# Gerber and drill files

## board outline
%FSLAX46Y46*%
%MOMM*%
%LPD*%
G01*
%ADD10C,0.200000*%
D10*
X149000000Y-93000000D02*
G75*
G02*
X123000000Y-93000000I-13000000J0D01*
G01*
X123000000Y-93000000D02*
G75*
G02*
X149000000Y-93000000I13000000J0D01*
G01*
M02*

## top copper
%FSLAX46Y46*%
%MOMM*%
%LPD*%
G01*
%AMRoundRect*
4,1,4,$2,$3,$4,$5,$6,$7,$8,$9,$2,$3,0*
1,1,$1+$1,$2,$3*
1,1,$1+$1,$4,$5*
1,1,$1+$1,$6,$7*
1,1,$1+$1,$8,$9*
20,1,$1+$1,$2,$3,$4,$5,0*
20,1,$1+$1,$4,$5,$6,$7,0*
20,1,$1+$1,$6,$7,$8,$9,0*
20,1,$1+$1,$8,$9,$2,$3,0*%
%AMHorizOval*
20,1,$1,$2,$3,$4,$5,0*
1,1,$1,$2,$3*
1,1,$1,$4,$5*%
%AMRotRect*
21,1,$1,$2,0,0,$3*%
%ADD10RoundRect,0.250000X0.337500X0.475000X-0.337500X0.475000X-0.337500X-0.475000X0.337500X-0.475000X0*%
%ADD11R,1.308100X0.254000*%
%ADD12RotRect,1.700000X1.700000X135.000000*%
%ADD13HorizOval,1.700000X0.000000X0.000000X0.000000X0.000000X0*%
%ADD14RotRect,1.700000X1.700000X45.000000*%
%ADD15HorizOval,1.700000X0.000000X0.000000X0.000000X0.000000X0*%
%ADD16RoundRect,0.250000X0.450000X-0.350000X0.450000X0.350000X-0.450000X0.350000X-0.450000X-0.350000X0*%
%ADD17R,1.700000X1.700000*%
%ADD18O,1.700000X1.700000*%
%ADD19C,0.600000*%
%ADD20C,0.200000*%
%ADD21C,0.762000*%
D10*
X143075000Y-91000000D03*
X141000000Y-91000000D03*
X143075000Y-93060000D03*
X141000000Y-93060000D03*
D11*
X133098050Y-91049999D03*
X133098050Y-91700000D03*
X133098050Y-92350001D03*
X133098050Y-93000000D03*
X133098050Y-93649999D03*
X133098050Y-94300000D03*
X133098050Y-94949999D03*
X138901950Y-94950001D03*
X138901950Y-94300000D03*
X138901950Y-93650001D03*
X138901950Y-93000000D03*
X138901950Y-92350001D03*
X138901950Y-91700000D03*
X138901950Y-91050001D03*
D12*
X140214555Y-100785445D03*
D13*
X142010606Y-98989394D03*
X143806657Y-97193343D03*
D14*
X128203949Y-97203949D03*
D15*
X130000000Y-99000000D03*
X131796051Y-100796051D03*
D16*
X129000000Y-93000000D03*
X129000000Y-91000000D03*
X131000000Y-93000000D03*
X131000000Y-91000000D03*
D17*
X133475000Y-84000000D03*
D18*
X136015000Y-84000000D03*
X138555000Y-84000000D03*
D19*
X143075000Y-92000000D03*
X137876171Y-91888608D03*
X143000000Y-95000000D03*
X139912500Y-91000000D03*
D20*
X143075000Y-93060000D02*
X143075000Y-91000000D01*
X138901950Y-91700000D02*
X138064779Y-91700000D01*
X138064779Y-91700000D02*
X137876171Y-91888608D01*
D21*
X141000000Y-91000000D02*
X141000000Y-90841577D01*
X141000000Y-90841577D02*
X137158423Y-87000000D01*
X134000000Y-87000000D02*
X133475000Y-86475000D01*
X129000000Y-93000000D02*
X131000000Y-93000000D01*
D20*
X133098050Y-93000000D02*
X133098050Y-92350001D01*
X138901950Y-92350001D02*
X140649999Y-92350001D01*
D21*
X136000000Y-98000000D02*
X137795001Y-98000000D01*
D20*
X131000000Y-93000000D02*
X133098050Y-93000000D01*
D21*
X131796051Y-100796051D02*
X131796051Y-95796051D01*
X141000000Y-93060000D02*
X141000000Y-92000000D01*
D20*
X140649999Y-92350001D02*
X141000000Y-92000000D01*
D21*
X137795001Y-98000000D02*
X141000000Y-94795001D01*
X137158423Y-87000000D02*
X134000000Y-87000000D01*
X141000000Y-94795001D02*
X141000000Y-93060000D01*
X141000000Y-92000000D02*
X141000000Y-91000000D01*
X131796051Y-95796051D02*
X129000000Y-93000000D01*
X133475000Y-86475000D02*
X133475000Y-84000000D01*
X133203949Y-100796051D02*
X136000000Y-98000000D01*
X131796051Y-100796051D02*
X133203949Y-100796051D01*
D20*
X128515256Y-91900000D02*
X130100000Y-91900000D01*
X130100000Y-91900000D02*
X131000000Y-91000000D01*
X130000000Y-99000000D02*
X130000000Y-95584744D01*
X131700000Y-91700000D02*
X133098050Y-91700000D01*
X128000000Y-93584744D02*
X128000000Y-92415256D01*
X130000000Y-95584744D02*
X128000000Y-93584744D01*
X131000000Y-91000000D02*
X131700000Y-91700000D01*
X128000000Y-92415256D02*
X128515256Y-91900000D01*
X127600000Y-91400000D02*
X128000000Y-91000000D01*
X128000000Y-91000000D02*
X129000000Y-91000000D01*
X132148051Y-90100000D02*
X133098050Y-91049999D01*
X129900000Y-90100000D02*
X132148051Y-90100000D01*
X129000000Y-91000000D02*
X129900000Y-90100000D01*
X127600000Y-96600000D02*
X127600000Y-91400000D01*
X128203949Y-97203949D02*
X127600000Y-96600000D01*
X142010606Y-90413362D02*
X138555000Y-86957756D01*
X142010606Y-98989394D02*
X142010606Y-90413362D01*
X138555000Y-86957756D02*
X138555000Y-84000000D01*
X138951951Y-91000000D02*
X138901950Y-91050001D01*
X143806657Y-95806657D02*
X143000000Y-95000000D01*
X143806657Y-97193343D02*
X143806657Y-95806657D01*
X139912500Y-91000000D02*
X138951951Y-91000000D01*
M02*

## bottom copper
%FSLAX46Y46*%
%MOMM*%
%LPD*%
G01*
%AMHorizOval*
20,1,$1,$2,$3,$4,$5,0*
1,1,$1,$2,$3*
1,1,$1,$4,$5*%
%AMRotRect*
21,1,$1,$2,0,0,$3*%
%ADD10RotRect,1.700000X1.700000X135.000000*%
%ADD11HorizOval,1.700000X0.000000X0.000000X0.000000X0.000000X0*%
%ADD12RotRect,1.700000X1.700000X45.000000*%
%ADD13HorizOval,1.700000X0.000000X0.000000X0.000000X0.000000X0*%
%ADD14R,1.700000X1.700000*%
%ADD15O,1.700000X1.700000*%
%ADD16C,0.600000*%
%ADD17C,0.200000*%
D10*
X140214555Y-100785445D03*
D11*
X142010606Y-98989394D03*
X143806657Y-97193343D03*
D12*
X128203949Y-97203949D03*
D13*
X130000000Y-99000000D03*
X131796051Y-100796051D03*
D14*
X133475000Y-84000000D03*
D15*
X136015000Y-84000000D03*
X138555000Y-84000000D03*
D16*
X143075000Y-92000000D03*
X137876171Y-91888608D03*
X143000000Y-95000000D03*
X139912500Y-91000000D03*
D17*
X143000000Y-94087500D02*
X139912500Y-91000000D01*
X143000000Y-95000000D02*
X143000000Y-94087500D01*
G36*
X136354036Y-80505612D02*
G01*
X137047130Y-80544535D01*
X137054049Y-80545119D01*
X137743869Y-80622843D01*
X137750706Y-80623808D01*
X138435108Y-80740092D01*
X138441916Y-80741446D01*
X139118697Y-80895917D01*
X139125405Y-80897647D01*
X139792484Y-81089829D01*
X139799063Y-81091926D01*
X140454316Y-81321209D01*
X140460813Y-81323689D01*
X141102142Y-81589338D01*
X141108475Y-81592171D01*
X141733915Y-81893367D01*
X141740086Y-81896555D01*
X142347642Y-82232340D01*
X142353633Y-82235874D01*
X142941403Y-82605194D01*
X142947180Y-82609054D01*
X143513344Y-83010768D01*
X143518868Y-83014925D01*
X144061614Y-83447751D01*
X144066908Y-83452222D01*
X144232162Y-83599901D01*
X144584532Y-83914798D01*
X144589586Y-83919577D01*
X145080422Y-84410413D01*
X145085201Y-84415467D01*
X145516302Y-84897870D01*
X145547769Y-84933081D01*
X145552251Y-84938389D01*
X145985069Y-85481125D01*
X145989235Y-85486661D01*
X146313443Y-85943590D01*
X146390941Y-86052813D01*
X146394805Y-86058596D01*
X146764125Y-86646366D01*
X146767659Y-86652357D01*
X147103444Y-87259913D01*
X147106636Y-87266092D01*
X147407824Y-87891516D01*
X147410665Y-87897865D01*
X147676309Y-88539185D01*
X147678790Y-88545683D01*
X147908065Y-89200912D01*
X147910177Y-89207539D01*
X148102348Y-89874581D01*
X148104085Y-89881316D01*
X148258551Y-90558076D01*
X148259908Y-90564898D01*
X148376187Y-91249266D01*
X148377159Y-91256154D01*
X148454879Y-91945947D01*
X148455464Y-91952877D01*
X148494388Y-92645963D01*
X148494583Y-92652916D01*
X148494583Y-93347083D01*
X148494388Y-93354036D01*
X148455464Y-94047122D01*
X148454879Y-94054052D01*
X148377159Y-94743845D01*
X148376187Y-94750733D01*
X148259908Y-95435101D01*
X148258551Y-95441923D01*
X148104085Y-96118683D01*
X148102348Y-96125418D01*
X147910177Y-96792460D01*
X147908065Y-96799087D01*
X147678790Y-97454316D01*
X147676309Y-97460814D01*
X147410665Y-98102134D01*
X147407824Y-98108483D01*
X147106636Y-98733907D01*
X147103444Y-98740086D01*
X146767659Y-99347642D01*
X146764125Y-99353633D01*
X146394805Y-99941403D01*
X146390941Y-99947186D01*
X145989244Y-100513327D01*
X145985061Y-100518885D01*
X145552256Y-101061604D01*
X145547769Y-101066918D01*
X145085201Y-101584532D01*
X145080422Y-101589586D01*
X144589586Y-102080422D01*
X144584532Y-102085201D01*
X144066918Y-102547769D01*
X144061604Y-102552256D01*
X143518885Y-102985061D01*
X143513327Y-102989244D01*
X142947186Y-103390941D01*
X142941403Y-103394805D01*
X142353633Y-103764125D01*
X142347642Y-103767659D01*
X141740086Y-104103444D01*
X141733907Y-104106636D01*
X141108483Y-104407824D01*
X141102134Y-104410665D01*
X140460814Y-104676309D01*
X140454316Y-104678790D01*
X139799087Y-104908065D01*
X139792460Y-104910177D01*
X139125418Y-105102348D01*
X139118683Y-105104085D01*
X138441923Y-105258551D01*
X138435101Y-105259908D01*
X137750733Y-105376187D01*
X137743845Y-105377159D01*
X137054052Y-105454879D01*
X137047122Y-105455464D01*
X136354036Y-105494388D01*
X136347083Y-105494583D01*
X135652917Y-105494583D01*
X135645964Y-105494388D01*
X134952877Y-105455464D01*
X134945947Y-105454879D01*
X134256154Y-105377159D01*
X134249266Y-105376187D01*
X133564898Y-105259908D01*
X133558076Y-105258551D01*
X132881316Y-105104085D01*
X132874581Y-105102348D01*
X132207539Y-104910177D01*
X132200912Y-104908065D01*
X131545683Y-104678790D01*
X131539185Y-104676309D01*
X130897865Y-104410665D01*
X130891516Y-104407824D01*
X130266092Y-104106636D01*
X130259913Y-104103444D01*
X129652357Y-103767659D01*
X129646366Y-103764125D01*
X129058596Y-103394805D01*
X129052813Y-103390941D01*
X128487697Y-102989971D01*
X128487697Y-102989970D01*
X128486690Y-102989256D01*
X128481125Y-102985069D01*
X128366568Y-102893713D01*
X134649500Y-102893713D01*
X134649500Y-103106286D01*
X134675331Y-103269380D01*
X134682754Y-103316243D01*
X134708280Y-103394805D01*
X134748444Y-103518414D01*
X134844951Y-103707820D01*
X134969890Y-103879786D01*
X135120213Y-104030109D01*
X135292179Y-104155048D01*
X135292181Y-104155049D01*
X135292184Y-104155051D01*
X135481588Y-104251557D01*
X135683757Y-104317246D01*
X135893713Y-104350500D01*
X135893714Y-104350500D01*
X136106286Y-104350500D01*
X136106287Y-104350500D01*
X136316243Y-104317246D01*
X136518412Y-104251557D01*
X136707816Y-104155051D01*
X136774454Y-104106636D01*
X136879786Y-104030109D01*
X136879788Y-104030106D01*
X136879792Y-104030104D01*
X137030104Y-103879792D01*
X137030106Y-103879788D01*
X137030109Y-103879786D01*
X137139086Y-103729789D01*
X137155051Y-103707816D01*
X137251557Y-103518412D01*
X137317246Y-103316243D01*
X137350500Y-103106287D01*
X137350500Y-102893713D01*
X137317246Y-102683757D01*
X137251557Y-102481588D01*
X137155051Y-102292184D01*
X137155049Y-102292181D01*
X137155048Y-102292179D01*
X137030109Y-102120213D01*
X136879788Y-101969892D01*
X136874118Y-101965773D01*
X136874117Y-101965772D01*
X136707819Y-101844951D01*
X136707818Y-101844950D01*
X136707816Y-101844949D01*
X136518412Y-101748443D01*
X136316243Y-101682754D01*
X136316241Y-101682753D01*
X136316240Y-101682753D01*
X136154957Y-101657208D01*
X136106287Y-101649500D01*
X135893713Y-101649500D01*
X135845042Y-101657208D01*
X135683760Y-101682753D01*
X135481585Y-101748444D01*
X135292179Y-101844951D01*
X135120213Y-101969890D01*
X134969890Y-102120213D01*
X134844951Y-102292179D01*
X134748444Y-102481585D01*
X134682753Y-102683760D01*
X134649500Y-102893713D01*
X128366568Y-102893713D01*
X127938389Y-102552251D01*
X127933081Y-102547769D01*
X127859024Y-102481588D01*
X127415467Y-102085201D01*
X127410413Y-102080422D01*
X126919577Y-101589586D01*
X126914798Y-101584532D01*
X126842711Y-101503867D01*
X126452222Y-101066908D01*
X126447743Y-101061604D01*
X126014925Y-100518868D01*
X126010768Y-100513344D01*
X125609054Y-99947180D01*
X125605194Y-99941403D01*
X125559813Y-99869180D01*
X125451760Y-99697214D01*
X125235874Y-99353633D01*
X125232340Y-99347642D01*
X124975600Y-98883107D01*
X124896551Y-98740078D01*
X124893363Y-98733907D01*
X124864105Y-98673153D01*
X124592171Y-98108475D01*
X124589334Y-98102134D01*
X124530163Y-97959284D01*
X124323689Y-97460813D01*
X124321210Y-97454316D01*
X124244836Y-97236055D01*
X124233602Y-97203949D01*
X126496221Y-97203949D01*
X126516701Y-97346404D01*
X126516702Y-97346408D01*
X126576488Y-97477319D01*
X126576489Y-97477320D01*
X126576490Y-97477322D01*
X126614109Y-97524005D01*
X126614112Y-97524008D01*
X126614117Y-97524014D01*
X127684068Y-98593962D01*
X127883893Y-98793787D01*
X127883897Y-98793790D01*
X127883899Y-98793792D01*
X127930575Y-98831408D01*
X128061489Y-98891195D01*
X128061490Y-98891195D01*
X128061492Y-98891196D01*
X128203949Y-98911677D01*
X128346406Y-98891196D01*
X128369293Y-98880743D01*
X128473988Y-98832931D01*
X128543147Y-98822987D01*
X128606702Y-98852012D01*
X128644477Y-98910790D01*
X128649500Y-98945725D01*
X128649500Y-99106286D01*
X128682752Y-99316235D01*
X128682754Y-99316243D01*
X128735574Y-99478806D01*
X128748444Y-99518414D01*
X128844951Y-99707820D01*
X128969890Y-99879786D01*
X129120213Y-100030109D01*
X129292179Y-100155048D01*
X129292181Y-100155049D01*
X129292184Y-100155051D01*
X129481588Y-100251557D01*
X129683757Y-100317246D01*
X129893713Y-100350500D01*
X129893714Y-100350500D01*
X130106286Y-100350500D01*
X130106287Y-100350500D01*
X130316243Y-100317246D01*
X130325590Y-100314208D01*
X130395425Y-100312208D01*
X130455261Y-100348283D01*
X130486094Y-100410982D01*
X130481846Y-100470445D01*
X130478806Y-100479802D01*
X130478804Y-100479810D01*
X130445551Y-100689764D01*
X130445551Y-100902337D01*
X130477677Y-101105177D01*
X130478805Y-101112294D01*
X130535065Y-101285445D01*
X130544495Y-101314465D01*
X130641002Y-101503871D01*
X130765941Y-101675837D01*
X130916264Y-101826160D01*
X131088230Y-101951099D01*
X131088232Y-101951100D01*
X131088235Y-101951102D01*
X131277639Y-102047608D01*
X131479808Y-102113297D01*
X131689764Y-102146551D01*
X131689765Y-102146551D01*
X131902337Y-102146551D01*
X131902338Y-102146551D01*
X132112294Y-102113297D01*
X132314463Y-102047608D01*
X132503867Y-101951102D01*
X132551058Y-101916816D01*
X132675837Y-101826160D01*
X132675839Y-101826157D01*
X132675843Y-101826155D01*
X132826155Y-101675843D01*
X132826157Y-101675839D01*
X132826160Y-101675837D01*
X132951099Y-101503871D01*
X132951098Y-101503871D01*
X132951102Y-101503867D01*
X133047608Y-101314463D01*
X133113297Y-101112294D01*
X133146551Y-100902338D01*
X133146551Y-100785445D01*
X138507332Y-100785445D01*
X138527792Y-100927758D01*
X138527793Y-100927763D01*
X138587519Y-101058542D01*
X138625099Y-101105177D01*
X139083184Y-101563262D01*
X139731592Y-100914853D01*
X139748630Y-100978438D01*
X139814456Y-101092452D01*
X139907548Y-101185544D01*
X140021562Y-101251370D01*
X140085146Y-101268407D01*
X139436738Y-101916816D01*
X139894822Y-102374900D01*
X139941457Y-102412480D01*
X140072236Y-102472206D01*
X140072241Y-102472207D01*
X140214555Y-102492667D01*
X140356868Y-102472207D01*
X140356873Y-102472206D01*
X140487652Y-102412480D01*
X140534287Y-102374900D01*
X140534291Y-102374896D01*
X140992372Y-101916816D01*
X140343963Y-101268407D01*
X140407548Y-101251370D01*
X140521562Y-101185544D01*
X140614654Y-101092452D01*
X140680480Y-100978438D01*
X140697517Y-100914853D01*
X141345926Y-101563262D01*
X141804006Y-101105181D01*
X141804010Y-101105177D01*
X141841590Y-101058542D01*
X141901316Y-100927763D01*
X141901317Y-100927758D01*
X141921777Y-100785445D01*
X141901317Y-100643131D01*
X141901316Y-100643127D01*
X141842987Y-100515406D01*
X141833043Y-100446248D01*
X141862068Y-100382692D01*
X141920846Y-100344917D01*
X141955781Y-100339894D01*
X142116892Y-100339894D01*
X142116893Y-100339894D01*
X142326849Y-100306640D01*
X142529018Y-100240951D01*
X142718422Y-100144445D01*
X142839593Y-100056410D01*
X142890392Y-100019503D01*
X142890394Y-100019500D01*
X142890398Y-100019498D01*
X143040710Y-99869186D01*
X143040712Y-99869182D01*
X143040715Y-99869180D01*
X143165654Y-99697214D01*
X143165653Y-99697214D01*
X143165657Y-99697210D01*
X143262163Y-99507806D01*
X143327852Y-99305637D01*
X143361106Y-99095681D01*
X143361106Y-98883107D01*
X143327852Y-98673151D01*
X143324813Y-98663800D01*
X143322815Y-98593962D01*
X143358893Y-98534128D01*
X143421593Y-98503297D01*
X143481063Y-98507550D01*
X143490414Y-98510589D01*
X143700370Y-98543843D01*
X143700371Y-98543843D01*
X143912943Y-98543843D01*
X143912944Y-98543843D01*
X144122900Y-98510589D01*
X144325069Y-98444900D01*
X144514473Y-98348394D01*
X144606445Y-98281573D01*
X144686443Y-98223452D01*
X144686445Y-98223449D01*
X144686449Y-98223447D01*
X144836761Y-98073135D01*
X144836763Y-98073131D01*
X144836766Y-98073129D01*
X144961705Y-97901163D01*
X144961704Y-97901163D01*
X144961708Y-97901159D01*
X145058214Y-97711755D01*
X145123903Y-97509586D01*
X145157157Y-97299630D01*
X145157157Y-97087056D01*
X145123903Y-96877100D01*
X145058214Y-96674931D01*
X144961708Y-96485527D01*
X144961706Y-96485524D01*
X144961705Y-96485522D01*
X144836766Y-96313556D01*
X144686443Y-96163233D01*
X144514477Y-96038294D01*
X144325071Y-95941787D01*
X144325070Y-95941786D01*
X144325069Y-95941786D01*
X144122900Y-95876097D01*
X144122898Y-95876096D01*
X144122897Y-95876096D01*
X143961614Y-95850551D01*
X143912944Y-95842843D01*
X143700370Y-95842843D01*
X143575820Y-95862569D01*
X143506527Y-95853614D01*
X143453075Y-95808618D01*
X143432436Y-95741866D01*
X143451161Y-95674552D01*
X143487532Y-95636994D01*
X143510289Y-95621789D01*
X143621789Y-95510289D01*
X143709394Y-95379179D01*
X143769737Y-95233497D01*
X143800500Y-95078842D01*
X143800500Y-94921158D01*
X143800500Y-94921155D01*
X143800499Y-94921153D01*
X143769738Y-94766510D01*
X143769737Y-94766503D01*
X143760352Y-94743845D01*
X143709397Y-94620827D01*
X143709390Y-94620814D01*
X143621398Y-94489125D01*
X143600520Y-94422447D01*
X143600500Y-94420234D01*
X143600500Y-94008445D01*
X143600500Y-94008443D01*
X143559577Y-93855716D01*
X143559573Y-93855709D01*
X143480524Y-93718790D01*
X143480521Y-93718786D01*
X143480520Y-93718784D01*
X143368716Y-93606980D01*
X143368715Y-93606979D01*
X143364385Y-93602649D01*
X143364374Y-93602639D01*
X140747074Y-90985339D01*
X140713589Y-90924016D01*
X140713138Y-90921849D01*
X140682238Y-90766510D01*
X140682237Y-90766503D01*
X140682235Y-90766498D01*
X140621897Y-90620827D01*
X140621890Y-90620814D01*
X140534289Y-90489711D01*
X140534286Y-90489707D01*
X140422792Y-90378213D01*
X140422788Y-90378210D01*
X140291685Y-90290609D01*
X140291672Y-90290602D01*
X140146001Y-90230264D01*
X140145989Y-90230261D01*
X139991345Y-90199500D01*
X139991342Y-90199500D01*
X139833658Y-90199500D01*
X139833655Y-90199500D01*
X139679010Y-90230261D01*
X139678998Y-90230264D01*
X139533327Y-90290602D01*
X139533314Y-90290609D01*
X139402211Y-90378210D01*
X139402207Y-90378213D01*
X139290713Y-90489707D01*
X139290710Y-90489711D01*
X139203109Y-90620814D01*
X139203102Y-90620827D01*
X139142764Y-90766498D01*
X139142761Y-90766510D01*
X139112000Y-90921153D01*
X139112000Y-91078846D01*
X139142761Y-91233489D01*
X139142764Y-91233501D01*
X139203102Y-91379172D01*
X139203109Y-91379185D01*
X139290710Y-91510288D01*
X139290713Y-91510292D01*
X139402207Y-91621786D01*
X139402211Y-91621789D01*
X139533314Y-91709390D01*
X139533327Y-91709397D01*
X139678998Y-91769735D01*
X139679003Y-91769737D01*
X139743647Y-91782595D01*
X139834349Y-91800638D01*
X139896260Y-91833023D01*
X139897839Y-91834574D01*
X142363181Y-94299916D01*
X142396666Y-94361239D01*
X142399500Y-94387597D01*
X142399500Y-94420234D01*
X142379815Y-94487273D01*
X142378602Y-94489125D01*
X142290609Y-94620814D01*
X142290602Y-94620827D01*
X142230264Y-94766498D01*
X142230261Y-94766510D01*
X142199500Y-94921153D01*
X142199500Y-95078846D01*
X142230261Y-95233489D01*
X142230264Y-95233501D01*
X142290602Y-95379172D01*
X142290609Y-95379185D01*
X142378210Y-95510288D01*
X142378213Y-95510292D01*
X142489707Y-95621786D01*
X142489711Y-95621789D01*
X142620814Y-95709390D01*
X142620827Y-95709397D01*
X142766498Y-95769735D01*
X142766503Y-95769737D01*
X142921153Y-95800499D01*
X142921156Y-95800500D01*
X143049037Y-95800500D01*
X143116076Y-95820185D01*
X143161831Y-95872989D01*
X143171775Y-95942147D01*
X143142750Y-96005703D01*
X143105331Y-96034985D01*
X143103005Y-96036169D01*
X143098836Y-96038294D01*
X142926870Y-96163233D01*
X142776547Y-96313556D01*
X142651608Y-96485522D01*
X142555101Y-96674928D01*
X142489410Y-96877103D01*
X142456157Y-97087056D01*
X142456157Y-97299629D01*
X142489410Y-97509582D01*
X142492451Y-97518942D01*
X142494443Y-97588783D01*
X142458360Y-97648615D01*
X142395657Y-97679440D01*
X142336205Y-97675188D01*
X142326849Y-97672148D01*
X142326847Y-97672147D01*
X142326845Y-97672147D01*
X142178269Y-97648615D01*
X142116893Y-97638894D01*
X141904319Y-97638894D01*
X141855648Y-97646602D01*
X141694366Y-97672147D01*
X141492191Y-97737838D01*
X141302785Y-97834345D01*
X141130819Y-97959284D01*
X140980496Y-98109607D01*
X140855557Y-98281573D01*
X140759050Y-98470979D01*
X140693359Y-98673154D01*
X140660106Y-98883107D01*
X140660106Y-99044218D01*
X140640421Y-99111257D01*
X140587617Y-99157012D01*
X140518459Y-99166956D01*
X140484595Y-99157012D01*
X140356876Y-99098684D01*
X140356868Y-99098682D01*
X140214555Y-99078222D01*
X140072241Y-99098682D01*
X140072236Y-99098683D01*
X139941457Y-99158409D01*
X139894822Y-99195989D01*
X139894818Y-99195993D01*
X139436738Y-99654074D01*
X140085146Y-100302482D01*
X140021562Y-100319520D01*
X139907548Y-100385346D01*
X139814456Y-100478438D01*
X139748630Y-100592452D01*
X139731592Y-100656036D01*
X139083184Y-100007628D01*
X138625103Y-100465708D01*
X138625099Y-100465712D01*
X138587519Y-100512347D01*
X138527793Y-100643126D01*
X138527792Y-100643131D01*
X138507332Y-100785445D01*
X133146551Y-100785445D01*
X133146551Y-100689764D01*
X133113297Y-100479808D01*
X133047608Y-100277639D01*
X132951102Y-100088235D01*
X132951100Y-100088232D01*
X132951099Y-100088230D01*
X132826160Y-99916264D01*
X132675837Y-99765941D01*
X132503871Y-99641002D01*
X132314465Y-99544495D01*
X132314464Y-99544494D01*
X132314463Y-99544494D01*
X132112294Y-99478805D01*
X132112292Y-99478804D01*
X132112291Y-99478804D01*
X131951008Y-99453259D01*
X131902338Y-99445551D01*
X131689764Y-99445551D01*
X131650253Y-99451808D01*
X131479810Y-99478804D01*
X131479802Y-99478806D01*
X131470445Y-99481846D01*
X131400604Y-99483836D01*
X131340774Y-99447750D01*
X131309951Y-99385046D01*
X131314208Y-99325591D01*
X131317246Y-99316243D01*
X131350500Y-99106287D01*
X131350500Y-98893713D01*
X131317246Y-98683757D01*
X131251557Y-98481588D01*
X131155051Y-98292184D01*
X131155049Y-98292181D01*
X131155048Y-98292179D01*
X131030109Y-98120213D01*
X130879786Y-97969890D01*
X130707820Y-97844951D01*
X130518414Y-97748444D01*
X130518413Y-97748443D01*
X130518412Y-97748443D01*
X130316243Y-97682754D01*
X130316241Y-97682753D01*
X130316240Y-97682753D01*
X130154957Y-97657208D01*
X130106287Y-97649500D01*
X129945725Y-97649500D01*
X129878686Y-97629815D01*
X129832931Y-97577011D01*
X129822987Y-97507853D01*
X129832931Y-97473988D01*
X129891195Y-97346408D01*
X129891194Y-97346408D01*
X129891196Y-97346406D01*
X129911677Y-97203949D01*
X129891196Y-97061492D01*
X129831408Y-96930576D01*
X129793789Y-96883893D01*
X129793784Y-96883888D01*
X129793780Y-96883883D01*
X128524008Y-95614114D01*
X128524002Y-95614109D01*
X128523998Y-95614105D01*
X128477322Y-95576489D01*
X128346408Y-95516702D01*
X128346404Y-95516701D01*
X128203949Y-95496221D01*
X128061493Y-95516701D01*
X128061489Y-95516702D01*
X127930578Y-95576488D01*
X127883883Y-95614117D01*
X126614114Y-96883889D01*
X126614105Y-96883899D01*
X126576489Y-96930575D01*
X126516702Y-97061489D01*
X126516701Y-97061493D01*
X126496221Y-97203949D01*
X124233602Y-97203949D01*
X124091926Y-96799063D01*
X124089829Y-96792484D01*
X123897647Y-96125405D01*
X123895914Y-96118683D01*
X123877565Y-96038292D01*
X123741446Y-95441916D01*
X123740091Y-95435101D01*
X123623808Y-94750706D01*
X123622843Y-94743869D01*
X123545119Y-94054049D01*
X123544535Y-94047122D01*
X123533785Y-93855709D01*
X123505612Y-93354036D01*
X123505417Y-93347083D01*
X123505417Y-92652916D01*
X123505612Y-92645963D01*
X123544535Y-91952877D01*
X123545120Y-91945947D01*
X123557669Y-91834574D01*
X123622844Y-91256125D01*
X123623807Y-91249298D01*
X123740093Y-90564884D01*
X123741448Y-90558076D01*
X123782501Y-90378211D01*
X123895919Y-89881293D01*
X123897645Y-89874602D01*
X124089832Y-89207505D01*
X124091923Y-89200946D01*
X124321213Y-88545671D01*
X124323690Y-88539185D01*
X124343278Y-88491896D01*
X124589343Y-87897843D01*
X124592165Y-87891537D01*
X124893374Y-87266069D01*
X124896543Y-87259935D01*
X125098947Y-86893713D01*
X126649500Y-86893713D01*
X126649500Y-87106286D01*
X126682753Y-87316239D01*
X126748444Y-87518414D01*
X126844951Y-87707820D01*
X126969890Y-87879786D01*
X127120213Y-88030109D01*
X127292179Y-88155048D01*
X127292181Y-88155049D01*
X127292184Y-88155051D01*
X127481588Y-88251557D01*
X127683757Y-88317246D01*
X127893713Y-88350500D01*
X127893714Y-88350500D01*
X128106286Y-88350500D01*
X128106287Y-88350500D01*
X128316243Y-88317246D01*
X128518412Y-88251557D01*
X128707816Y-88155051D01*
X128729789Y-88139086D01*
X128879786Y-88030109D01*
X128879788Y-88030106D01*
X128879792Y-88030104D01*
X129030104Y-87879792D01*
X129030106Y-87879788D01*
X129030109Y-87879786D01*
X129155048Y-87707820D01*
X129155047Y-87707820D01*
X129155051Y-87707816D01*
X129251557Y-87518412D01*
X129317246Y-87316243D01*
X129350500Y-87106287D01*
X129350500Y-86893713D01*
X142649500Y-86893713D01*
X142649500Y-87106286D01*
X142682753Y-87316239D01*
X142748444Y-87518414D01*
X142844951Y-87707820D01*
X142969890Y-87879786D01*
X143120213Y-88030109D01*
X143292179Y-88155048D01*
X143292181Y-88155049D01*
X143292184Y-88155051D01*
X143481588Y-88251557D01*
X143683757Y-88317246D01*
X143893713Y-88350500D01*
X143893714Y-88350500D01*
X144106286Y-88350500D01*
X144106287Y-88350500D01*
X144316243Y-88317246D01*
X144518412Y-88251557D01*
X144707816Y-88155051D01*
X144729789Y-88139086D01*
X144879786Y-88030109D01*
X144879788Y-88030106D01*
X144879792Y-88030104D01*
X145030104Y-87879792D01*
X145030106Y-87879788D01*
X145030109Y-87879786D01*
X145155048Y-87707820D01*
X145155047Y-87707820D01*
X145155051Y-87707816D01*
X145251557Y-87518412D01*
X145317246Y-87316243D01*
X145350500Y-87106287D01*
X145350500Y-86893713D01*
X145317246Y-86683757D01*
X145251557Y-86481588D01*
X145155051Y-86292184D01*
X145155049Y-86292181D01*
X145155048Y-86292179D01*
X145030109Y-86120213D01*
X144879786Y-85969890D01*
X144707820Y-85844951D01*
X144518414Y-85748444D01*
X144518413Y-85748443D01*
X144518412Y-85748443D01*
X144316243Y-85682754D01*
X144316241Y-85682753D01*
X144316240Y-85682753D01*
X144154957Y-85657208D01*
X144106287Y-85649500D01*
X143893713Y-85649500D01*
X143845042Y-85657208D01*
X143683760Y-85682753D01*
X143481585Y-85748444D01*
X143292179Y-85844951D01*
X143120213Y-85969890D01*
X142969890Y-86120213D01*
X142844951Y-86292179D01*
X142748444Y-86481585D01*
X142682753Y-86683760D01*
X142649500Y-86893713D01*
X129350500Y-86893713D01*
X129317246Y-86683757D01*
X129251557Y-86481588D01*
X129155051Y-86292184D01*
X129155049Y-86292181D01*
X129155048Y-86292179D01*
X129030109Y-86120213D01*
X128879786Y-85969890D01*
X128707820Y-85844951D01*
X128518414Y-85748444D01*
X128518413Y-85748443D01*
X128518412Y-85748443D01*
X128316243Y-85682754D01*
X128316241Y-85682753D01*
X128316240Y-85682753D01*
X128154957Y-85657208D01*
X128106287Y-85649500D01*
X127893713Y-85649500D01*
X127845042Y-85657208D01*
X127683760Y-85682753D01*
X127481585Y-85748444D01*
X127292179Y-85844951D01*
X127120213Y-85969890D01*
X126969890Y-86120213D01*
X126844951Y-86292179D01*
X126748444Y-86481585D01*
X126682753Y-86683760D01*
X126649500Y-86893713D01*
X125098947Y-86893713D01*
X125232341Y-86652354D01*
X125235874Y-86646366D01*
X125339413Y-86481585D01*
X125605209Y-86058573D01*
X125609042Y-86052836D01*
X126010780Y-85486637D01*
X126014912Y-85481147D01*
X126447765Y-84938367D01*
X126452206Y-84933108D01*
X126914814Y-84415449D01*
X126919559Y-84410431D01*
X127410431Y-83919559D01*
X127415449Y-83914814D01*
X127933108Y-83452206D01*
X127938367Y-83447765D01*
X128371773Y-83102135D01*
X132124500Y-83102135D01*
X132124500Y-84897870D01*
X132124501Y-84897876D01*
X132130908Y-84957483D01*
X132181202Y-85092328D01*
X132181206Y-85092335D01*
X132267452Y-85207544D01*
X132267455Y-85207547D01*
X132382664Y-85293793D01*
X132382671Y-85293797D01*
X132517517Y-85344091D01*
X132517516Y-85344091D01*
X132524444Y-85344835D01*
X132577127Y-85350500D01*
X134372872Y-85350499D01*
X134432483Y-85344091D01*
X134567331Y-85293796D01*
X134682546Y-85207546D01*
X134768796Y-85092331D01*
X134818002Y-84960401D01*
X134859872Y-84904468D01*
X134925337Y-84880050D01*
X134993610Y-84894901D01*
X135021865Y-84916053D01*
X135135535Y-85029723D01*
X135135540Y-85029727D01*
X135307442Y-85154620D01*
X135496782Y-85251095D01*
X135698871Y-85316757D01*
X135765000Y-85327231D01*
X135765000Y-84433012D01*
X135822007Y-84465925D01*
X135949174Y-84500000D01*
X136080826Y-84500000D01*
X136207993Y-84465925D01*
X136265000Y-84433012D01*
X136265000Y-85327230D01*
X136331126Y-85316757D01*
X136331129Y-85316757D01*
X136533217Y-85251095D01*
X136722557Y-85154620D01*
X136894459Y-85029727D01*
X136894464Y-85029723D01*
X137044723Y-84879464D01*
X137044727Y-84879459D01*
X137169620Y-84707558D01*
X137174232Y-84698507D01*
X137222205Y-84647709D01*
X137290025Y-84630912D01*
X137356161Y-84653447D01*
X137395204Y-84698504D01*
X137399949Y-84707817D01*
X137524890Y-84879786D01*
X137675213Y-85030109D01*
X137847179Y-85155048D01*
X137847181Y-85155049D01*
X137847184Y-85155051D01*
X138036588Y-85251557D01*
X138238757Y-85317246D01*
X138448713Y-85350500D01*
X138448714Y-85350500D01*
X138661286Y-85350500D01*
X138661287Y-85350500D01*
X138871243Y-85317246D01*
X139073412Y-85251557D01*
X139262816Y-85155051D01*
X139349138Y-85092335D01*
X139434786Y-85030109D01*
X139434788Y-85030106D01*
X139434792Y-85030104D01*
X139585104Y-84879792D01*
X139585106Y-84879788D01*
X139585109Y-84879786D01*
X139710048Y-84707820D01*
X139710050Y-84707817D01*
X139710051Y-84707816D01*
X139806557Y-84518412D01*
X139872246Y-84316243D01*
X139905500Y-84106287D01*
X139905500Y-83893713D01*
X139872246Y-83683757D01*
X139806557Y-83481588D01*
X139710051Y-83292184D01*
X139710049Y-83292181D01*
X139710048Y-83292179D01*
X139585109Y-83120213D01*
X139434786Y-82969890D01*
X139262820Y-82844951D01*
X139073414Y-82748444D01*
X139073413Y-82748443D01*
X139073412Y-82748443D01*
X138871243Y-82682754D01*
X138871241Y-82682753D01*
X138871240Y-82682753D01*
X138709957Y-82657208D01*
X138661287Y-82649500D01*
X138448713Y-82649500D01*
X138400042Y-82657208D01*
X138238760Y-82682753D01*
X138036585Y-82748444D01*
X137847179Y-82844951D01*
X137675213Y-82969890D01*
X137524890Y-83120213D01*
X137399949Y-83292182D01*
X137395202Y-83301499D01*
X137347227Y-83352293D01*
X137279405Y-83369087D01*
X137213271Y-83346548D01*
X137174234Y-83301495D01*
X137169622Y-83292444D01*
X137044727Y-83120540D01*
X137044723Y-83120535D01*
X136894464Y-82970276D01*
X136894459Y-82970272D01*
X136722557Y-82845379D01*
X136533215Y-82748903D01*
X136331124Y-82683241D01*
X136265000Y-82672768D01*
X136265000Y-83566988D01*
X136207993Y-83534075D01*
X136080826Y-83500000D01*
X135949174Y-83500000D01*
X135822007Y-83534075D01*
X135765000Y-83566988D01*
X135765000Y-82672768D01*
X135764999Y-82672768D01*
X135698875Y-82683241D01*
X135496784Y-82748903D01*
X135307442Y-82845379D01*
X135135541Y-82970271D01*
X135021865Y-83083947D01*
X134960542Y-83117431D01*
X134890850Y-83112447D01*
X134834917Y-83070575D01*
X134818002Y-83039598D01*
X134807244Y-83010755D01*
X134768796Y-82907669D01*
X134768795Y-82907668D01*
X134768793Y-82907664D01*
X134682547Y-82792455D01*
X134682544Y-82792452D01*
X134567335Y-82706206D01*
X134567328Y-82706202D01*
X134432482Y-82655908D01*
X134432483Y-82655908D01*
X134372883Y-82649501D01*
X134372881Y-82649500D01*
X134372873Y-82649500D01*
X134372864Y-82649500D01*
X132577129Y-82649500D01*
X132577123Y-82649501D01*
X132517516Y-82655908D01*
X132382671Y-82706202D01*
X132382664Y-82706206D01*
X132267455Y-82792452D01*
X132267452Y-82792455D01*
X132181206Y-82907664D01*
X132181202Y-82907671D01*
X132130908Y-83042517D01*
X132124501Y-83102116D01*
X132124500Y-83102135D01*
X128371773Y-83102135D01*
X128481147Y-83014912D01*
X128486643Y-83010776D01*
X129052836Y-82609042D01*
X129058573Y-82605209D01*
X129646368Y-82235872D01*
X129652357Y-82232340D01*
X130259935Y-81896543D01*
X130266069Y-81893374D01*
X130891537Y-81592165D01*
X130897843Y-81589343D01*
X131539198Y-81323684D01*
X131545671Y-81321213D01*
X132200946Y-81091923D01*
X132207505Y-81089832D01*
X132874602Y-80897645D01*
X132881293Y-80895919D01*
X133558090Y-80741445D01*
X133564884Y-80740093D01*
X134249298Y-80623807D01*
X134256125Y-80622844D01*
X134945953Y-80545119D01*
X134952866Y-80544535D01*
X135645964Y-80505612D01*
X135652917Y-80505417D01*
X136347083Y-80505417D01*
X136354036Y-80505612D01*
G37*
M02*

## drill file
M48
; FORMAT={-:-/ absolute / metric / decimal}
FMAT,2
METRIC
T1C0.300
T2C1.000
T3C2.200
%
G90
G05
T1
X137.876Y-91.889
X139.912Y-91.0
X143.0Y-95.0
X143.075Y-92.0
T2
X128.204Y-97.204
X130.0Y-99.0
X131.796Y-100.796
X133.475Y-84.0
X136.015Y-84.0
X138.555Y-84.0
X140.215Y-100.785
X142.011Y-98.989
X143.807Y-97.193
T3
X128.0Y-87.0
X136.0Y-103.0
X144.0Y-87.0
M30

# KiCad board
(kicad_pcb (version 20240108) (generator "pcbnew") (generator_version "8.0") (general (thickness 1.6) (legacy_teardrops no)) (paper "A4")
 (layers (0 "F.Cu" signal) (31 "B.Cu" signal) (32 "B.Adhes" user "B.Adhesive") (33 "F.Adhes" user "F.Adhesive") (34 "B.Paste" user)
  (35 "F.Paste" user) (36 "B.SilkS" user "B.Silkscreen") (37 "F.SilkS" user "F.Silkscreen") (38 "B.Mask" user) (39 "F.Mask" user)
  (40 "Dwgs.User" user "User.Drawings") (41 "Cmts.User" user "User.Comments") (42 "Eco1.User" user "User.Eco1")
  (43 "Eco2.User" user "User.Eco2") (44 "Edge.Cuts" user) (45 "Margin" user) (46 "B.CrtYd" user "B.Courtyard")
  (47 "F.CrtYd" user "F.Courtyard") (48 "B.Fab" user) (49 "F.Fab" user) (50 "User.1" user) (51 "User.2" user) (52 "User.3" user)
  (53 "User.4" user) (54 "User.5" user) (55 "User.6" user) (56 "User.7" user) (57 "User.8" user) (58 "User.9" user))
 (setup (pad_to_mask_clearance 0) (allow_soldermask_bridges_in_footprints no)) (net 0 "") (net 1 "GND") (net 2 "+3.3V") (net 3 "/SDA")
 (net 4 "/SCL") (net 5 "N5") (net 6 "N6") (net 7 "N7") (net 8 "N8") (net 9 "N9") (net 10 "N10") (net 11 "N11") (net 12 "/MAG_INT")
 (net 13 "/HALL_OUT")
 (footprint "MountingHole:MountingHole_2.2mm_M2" (layer "F.Cu") (at 128 87)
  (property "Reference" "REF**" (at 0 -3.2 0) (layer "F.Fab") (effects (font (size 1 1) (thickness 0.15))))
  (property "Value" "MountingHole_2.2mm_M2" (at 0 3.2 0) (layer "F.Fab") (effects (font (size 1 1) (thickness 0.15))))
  (pad "" np_thru_hole circle (at 0 0) (size 2.2 2.2) (drill 2.2) (layers "*.Cu" "*.Mask")))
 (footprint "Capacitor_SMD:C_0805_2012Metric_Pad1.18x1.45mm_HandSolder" (layer "F.Cu") (at 142.0375 91 180)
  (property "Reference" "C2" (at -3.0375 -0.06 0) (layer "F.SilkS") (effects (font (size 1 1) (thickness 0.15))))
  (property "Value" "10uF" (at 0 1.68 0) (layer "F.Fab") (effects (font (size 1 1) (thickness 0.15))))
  (pad "1" smd roundrect (at -1.0375 0 180) (size 1.175 1.45) (layers "F.Cu" "F.Paste" "F.Mask") (roundrect_rratio 0.212766) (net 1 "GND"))
  (pad "2" smd roundrect (at 1.0375 0 180) (size 1.175 1.45) (layers "F.Cu" "F.Paste" "F.Mask") (roundrect_rratio 0.212766) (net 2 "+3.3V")))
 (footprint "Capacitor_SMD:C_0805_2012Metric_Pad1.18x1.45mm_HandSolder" (layer "F.Cu") (at 142.0375 93.06 180)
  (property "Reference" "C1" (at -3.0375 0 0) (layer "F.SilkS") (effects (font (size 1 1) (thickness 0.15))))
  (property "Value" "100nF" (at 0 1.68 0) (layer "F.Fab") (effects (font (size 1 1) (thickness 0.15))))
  (pad "1" smd roundrect (at -1.0375 0 180) (size 1.175 1.45) (layers "F.Cu" "F.Paste" "F.Mask") (roundrect_rratio 0.212766) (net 1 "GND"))
  (pad "2" smd roundrect (at 1.0375 0 180) (size 1.175 1.45) (layers "F.Cu" "F.Paste" "F.Mask") (roundrect_rratio 0.212766) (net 2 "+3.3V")))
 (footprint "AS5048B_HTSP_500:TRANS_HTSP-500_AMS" (layer "F.Cu") (at 136 93)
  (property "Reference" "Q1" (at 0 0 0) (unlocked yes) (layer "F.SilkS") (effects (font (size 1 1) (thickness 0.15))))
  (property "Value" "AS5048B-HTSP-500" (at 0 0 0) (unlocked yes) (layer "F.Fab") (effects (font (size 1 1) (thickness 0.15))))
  (pad "1" smd rect (at -2.90195 -1.950001) (size 1.3081 0.254) (layers "F.Cu" "F.Paste" "F.Mask") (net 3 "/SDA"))
  (pad "2" smd rect (at -2.90195 -1.3) (size 1.3081 0.254) (layers "F.Cu" "F.Paste" "F.Mask") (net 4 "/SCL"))
  (pad "3" smd rect (at -2.90195 -0.649999) (size 1.3081 0.254) (layers "F.Cu" "F.Paste" "F.Mask") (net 2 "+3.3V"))
  (pad "4" smd rect (at -2.90195 0) (size 1.3081 0.254) (layers "F.Cu" "F.Paste" "F.Mask") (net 2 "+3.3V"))
  (pad "5" smd rect (at -2.90195 0.649999) (size 1.3081 0.254) (layers "F.Cu" "F.Paste" "F.Mask") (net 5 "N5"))
  (pad "6" smd rect (at -2.90195 1.3) (size 1.3081 0.254) (layers "F.Cu" "F.Paste" "F.Mask") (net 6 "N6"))
  (pad "7" smd rect (at -2.90195 1.949999) (size 1.3081 0.254) (layers "F.Cu" "F.Paste" "F.Mask") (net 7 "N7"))
  (pad "8" smd rect (at 2.90195 1.950001) (size 1.3081 0.254) (layers "F.Cu" "F.Paste" "F.Mask") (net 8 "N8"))
  (pad "9" smd rect (at 2.90195 1.3) (size 1.3081 0.254) (layers "F.Cu" "F.Paste" "F.Mask") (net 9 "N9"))
  (pad "10" smd rect (at 2.90195 0.650001) (size 1.3081 0.254) (layers "F.Cu" "F.Paste" "F.Mask") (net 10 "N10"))
  (pad "11" smd rect (at 2.90195 0) (size 1.3081 0.254) (layers "F.Cu" "F.Paste" "F.Mask") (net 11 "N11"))
  (pad "12" smd rect (at 2.90195 -0.649999) (size 1.3081 0.254) (layers "F.Cu" "F.Paste" "F.Mask") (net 2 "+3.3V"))
  (pad "13" smd rect (at 2.90195 -1.3) (size 1.3081 0.254) (layers "F.Cu" "F.Paste" "F.Mask") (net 1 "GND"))
  (pad "14" smd rect (at 2.90195 -1.949999) (size 1.3081 0.254) (layers "F.Cu" "F.Paste" "F.Mask") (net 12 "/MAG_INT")))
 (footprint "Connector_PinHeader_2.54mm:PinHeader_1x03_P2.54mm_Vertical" (layer "F.Cu") (at 140.214555 100.785445 135)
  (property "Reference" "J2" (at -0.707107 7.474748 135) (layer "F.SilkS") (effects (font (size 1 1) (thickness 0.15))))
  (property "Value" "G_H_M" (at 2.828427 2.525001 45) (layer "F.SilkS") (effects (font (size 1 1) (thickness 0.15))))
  (pad "1" thru_hole rect (at 0 0 135) (size 1.7 1.7) (drill 1) (layers "*.Cu" "*.Mask") (remove_unused_layers no) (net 1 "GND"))
  (pad "2" thru_hole oval (at 0 2.54 135) (size 1.7 1.7) (drill 1) (layers "*.Cu" "*.Mask") (remove_unused_layers no) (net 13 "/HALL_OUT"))
  (pad "3" thru_hole oval (at 0 5.079999 135) (size 1.7 1.7) (drill 1) (layers "*.Cu" "*.Mask") (remove_unused_layers no)
   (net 12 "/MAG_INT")))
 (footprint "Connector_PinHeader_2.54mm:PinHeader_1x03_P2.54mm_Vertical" (layer "F.Cu") (at 128.203949 97.203949 45)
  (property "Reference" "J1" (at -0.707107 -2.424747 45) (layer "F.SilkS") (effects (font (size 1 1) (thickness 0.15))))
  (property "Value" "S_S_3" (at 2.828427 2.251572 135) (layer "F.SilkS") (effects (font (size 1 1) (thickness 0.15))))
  (pad "1" thru_hole rect (at 0 0 45) (size 1.7 1.7) (drill 1) (layers "*.Cu" "*.Mask") (remove_unused_layers no) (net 3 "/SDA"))
  (pad "2" thru_hole oval (at 0 2.54 45) (size 1.7 1.7) (drill 1) (layers "*.Cu" "*.Mask") (remove_unused_layers no) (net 4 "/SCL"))
  (pad "3" thru_hole oval (at 0 5.079999 45) (size 1.7 1.7) (drill 1) (layers "*.Cu" "*.Mask") (remove_unused_layers no) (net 2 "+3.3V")))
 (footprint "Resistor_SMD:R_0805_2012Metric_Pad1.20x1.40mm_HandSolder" (layer "F.Cu") (at 129 92 90)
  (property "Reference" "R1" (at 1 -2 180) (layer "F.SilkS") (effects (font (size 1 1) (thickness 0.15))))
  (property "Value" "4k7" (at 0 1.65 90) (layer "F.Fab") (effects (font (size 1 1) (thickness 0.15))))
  (pad "1" smd roundrect (at -1 0 90) (size 1.2 1.4) (layers "F.Cu" "F.Paste" "F.Mask") (roundrect_rratio 0.208333) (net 2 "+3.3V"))
  (pad "2" smd roundrect (at 1 0 90) (size 1.2 1.4) (layers "F.Cu" "F.Paste" "F.Mask") (roundrect_rratio 0.208333) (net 3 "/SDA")))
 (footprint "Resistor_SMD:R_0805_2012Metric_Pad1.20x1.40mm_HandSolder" (layer "F.Cu") (at 131 92 90)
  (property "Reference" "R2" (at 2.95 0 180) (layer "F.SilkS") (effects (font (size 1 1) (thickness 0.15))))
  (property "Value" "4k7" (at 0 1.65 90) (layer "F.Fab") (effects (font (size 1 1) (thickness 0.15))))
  (pad "1" smd roundrect (at -1 0 90) (size 1.2 1.4) (layers "F.Cu" "F.Paste" "F.Mask") (roundrect_rratio 0.208333) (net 2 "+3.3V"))
  (pad "2" smd roundrect (at 1 0 90) (size 1.2 1.4) (layers "F.Cu" "F.Paste" "F.Mask") (roundrect_rratio 0.208333) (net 4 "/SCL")))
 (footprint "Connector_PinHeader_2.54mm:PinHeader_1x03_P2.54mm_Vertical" (layer "F.Cu") (at 133.475 84 90)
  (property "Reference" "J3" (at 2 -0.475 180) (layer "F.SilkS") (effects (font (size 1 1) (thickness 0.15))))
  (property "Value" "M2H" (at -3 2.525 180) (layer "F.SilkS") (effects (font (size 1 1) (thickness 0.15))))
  (pad "1" thru_hole rect (at 0 0 90) (size 1.7 1.7) (drill 1) (layers "*.Cu" "*.Mask") (remove_unused_layers no) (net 2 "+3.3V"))
  (pad "2" thru_hole oval (at 0 2.54 90) (size 1.7 1.7) (drill 1) (layers "*.Cu" "*.Mask") (remove_unused_layers no) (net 1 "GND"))
  (pad "3" thru_hole oval (at 0 5.08 90) (size 1.7 1.7) (drill 1) (layers "*.Cu" "*.Mask") (remove_unused_layers no) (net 13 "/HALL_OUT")))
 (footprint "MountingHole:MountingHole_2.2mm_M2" (layer "F.Cu") (at 144 87)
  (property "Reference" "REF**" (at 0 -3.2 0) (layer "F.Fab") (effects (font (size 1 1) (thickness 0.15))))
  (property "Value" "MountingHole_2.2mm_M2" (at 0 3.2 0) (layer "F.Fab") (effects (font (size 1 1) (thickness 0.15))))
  (pad "" np_thru_hole circle (at 0 0) (size 2.2 2.2) (drill 2.2) (layers "*.Cu" "*.Mask")))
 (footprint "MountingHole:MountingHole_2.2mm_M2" (layer "F.Cu") (at 136 103)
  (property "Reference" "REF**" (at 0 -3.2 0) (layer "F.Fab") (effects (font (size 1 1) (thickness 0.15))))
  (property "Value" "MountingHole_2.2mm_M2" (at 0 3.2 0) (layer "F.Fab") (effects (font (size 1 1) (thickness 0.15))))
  (pad "" np_thru_hole circle (at 0 0) (size 2.2 2.2) (drill 2.2) (layers "*.Cu" "*.Mask")))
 (gr_circle (center 136 93) (end 149 93) (stroke (width 0.2) (type default)) (fill none) (layer "Edge.Cuts"))
 (segment (start 143.075 93.06) (end 143.075 91) (width 0.2) (layer "F.Cu") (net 1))
 (segment (start 138.90195 91.7) (end 138.064779 91.7) (width 0.2) (layer "F.Cu") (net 1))
 (segment (start 138.064779 91.7) (end 137.876171 91.888608) (width 0.2) (layer "F.Cu") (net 1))
 (via (at 143.075 92) (size 0.6) (drill 0.3) (layers "F.Cu" "B.Cu") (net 1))
 (via (at 137.876171 91.888608) (size 0.6) (drill 0.3) (layers "F.Cu" "B.Cu") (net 1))
 (segment (start 141 91) (end 141 90.841577) (width 0.762) (layer "F.Cu") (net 2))
 (segment (start 141 90.841577) (end 137.158423 87) (width 0.762) (layer "F.Cu") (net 2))
 (segment (start 134 87) (end 133.475 86.475) (width 0.762) (layer "F.Cu") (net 2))
 (segment (start 129 93) (end 131 93) (width 0.762) (layer "F.Cu") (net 2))
 (segment (start 133.09805 93) (end 133.09805 92.350001) (width 0.2) (layer "F.Cu") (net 2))
 (segment (start 138.90195 92.350001) (end 140.649999 92.350001) (width 0.2) (layer "F.Cu") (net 2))
 (segment (start 136 98) (end 137.795001 98) (width 0.762) (layer "F.Cu") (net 2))
 (segment (start 131 93) (end 133.09805 93) (width 0.2) (layer "F.Cu") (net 2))
 (segment (start 131.796051 100.796051) (end 131.796051 95.796051) (width 0.762) (layer "F.Cu") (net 2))
 (segment (start 141 93.06) (end 141 92) (width 0.762) (layer "F.Cu") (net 2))
 (segment (start 140.649999 92.350001) (end 141 92) (width 0.2) (layer "F.Cu") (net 2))
 (segment (start 137.795001 98) (end 141 94.795001) (width 0.762) (layer "F.Cu") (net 2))
 (segment (start 137.158423 87) (end 134 87) (width 0.762) (layer "F.Cu") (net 2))
 (segment (start 141 94.795001) (end 141 93.06) (width 0.762) (layer "F.Cu") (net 2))
 (segment (start 141 92) (end 141 91) (width 0.762) (layer "F.Cu") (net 2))
 (segment (start 131.796051 95.796051) (end 129 93) (width 0.762) (layer "F.Cu") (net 2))
 (segment (start 133.475 86.475) (end 133.475 84) (width 0.762) (layer "F.Cu") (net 2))
 (segment (start 133.203949 100.796051) (end 136 98) (width 0.762) (layer "F.Cu") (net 2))
 (segment (start 131.796051 100.796051) (end 133.203949 100.796051) (width 0.762) (layer "F.Cu") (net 2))
 (segment (start 128.515256 91.9) (end 130.1 91.9) (width 0.2) (layer "F.Cu") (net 4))
 (segment (start 130.1 91.9) (end 131 91) (width 0.2) (layer "F.Cu") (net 4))
 (segment (start 130 99) (end 130 95.584744) (width 0.2) (layer "F.Cu") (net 4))
 (segment (start 131.7 91.7) (end 133.09805 91.7) (width 0.2) (layer "F.Cu") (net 4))
 (segment (start 128 93.584744) (end 128 92.415256) (width 0.2) (layer "F.Cu") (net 4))
 (segment (start 130 95.584744) (end 128 93.584744) (width 0.2) (layer "F.Cu") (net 4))
 (segment (start 131 91) (end 131.7 91.7) (width 0.2) (layer "F.Cu") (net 4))
 (segment (start 128 92.415256) (end 128.515256 91.9) (width 0.2) (layer "F.Cu") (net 4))
 (segment (start 127.6 91.4) (end 128 91) (width 0.2) (layer "F.Cu") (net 3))
 (segment (start 128 91) (end 129 91) (width 0.2) (layer "F.Cu") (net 3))
 (segment (start 132.148051 90.1) (end 133.09805 91.049999) (width 0.2) (layer "F.Cu") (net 3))
 (segment (start 129.9 90.1) (end 132.148051 90.1) (width 0.2) (layer "F.Cu") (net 3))
 (segment (start 129 91) (end 129.9 90.1) (width 0.2) (layer "F.Cu") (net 3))
 (segment (start 127.6 96.6) (end 127.6 91.4) (width 0.2) (layer "F.Cu") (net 3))
 (segment (start 128.203949 97.203949) (end 127.6 96.6) (width 0.2) (layer "F.Cu") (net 3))
 (segment (start 142.010606 90.413362) (end 138.555 86.957756) (width 0.2) (layer "F.Cu") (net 13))
 (segment (start 142.010606 98.989394) (end 142.010606 90.413362) (width 0.2) (layer "F.Cu") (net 13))
 (segment (start 138.555 86.957756) (end 138.555 84) (width 0.2) (layer "F.Cu") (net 13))
 (segment (start 138.951951 91) (end 138.90195 91.050001) (width 0.2) (layer "F.Cu") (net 12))
 (segment (start 143.806657 95.806657) (end 143 95) (width 0.2) (layer "F.Cu") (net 12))
 (segment (start 143.806657 97.193343) (end 143.806657 95.806657) (width 0.2) (layer "F.Cu") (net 12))
 (segment (start 139.9125 91) (end 138.951951 91) (width 0.2) (layer "F.Cu") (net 12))
 (via (at 143 95) (size 0.6) (drill 0.3) (layers "F.Cu" "B.Cu") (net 12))
 (via (at 139.9125 91) (size 0.6) (drill 0.3) (layers "F.Cu" "B.Cu") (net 12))
 (segment (start 143 94.0875) (end 139.9125 91) (width 0.2) (layer "B.Cu") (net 12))
 (segment (start 143 95) (end 143 94.0875) (width 0.2) (layer "B.Cu") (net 12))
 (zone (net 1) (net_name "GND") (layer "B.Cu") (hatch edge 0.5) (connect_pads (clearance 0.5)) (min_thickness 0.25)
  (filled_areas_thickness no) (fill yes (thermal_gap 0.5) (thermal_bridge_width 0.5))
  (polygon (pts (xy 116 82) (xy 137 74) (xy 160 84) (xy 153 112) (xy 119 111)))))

